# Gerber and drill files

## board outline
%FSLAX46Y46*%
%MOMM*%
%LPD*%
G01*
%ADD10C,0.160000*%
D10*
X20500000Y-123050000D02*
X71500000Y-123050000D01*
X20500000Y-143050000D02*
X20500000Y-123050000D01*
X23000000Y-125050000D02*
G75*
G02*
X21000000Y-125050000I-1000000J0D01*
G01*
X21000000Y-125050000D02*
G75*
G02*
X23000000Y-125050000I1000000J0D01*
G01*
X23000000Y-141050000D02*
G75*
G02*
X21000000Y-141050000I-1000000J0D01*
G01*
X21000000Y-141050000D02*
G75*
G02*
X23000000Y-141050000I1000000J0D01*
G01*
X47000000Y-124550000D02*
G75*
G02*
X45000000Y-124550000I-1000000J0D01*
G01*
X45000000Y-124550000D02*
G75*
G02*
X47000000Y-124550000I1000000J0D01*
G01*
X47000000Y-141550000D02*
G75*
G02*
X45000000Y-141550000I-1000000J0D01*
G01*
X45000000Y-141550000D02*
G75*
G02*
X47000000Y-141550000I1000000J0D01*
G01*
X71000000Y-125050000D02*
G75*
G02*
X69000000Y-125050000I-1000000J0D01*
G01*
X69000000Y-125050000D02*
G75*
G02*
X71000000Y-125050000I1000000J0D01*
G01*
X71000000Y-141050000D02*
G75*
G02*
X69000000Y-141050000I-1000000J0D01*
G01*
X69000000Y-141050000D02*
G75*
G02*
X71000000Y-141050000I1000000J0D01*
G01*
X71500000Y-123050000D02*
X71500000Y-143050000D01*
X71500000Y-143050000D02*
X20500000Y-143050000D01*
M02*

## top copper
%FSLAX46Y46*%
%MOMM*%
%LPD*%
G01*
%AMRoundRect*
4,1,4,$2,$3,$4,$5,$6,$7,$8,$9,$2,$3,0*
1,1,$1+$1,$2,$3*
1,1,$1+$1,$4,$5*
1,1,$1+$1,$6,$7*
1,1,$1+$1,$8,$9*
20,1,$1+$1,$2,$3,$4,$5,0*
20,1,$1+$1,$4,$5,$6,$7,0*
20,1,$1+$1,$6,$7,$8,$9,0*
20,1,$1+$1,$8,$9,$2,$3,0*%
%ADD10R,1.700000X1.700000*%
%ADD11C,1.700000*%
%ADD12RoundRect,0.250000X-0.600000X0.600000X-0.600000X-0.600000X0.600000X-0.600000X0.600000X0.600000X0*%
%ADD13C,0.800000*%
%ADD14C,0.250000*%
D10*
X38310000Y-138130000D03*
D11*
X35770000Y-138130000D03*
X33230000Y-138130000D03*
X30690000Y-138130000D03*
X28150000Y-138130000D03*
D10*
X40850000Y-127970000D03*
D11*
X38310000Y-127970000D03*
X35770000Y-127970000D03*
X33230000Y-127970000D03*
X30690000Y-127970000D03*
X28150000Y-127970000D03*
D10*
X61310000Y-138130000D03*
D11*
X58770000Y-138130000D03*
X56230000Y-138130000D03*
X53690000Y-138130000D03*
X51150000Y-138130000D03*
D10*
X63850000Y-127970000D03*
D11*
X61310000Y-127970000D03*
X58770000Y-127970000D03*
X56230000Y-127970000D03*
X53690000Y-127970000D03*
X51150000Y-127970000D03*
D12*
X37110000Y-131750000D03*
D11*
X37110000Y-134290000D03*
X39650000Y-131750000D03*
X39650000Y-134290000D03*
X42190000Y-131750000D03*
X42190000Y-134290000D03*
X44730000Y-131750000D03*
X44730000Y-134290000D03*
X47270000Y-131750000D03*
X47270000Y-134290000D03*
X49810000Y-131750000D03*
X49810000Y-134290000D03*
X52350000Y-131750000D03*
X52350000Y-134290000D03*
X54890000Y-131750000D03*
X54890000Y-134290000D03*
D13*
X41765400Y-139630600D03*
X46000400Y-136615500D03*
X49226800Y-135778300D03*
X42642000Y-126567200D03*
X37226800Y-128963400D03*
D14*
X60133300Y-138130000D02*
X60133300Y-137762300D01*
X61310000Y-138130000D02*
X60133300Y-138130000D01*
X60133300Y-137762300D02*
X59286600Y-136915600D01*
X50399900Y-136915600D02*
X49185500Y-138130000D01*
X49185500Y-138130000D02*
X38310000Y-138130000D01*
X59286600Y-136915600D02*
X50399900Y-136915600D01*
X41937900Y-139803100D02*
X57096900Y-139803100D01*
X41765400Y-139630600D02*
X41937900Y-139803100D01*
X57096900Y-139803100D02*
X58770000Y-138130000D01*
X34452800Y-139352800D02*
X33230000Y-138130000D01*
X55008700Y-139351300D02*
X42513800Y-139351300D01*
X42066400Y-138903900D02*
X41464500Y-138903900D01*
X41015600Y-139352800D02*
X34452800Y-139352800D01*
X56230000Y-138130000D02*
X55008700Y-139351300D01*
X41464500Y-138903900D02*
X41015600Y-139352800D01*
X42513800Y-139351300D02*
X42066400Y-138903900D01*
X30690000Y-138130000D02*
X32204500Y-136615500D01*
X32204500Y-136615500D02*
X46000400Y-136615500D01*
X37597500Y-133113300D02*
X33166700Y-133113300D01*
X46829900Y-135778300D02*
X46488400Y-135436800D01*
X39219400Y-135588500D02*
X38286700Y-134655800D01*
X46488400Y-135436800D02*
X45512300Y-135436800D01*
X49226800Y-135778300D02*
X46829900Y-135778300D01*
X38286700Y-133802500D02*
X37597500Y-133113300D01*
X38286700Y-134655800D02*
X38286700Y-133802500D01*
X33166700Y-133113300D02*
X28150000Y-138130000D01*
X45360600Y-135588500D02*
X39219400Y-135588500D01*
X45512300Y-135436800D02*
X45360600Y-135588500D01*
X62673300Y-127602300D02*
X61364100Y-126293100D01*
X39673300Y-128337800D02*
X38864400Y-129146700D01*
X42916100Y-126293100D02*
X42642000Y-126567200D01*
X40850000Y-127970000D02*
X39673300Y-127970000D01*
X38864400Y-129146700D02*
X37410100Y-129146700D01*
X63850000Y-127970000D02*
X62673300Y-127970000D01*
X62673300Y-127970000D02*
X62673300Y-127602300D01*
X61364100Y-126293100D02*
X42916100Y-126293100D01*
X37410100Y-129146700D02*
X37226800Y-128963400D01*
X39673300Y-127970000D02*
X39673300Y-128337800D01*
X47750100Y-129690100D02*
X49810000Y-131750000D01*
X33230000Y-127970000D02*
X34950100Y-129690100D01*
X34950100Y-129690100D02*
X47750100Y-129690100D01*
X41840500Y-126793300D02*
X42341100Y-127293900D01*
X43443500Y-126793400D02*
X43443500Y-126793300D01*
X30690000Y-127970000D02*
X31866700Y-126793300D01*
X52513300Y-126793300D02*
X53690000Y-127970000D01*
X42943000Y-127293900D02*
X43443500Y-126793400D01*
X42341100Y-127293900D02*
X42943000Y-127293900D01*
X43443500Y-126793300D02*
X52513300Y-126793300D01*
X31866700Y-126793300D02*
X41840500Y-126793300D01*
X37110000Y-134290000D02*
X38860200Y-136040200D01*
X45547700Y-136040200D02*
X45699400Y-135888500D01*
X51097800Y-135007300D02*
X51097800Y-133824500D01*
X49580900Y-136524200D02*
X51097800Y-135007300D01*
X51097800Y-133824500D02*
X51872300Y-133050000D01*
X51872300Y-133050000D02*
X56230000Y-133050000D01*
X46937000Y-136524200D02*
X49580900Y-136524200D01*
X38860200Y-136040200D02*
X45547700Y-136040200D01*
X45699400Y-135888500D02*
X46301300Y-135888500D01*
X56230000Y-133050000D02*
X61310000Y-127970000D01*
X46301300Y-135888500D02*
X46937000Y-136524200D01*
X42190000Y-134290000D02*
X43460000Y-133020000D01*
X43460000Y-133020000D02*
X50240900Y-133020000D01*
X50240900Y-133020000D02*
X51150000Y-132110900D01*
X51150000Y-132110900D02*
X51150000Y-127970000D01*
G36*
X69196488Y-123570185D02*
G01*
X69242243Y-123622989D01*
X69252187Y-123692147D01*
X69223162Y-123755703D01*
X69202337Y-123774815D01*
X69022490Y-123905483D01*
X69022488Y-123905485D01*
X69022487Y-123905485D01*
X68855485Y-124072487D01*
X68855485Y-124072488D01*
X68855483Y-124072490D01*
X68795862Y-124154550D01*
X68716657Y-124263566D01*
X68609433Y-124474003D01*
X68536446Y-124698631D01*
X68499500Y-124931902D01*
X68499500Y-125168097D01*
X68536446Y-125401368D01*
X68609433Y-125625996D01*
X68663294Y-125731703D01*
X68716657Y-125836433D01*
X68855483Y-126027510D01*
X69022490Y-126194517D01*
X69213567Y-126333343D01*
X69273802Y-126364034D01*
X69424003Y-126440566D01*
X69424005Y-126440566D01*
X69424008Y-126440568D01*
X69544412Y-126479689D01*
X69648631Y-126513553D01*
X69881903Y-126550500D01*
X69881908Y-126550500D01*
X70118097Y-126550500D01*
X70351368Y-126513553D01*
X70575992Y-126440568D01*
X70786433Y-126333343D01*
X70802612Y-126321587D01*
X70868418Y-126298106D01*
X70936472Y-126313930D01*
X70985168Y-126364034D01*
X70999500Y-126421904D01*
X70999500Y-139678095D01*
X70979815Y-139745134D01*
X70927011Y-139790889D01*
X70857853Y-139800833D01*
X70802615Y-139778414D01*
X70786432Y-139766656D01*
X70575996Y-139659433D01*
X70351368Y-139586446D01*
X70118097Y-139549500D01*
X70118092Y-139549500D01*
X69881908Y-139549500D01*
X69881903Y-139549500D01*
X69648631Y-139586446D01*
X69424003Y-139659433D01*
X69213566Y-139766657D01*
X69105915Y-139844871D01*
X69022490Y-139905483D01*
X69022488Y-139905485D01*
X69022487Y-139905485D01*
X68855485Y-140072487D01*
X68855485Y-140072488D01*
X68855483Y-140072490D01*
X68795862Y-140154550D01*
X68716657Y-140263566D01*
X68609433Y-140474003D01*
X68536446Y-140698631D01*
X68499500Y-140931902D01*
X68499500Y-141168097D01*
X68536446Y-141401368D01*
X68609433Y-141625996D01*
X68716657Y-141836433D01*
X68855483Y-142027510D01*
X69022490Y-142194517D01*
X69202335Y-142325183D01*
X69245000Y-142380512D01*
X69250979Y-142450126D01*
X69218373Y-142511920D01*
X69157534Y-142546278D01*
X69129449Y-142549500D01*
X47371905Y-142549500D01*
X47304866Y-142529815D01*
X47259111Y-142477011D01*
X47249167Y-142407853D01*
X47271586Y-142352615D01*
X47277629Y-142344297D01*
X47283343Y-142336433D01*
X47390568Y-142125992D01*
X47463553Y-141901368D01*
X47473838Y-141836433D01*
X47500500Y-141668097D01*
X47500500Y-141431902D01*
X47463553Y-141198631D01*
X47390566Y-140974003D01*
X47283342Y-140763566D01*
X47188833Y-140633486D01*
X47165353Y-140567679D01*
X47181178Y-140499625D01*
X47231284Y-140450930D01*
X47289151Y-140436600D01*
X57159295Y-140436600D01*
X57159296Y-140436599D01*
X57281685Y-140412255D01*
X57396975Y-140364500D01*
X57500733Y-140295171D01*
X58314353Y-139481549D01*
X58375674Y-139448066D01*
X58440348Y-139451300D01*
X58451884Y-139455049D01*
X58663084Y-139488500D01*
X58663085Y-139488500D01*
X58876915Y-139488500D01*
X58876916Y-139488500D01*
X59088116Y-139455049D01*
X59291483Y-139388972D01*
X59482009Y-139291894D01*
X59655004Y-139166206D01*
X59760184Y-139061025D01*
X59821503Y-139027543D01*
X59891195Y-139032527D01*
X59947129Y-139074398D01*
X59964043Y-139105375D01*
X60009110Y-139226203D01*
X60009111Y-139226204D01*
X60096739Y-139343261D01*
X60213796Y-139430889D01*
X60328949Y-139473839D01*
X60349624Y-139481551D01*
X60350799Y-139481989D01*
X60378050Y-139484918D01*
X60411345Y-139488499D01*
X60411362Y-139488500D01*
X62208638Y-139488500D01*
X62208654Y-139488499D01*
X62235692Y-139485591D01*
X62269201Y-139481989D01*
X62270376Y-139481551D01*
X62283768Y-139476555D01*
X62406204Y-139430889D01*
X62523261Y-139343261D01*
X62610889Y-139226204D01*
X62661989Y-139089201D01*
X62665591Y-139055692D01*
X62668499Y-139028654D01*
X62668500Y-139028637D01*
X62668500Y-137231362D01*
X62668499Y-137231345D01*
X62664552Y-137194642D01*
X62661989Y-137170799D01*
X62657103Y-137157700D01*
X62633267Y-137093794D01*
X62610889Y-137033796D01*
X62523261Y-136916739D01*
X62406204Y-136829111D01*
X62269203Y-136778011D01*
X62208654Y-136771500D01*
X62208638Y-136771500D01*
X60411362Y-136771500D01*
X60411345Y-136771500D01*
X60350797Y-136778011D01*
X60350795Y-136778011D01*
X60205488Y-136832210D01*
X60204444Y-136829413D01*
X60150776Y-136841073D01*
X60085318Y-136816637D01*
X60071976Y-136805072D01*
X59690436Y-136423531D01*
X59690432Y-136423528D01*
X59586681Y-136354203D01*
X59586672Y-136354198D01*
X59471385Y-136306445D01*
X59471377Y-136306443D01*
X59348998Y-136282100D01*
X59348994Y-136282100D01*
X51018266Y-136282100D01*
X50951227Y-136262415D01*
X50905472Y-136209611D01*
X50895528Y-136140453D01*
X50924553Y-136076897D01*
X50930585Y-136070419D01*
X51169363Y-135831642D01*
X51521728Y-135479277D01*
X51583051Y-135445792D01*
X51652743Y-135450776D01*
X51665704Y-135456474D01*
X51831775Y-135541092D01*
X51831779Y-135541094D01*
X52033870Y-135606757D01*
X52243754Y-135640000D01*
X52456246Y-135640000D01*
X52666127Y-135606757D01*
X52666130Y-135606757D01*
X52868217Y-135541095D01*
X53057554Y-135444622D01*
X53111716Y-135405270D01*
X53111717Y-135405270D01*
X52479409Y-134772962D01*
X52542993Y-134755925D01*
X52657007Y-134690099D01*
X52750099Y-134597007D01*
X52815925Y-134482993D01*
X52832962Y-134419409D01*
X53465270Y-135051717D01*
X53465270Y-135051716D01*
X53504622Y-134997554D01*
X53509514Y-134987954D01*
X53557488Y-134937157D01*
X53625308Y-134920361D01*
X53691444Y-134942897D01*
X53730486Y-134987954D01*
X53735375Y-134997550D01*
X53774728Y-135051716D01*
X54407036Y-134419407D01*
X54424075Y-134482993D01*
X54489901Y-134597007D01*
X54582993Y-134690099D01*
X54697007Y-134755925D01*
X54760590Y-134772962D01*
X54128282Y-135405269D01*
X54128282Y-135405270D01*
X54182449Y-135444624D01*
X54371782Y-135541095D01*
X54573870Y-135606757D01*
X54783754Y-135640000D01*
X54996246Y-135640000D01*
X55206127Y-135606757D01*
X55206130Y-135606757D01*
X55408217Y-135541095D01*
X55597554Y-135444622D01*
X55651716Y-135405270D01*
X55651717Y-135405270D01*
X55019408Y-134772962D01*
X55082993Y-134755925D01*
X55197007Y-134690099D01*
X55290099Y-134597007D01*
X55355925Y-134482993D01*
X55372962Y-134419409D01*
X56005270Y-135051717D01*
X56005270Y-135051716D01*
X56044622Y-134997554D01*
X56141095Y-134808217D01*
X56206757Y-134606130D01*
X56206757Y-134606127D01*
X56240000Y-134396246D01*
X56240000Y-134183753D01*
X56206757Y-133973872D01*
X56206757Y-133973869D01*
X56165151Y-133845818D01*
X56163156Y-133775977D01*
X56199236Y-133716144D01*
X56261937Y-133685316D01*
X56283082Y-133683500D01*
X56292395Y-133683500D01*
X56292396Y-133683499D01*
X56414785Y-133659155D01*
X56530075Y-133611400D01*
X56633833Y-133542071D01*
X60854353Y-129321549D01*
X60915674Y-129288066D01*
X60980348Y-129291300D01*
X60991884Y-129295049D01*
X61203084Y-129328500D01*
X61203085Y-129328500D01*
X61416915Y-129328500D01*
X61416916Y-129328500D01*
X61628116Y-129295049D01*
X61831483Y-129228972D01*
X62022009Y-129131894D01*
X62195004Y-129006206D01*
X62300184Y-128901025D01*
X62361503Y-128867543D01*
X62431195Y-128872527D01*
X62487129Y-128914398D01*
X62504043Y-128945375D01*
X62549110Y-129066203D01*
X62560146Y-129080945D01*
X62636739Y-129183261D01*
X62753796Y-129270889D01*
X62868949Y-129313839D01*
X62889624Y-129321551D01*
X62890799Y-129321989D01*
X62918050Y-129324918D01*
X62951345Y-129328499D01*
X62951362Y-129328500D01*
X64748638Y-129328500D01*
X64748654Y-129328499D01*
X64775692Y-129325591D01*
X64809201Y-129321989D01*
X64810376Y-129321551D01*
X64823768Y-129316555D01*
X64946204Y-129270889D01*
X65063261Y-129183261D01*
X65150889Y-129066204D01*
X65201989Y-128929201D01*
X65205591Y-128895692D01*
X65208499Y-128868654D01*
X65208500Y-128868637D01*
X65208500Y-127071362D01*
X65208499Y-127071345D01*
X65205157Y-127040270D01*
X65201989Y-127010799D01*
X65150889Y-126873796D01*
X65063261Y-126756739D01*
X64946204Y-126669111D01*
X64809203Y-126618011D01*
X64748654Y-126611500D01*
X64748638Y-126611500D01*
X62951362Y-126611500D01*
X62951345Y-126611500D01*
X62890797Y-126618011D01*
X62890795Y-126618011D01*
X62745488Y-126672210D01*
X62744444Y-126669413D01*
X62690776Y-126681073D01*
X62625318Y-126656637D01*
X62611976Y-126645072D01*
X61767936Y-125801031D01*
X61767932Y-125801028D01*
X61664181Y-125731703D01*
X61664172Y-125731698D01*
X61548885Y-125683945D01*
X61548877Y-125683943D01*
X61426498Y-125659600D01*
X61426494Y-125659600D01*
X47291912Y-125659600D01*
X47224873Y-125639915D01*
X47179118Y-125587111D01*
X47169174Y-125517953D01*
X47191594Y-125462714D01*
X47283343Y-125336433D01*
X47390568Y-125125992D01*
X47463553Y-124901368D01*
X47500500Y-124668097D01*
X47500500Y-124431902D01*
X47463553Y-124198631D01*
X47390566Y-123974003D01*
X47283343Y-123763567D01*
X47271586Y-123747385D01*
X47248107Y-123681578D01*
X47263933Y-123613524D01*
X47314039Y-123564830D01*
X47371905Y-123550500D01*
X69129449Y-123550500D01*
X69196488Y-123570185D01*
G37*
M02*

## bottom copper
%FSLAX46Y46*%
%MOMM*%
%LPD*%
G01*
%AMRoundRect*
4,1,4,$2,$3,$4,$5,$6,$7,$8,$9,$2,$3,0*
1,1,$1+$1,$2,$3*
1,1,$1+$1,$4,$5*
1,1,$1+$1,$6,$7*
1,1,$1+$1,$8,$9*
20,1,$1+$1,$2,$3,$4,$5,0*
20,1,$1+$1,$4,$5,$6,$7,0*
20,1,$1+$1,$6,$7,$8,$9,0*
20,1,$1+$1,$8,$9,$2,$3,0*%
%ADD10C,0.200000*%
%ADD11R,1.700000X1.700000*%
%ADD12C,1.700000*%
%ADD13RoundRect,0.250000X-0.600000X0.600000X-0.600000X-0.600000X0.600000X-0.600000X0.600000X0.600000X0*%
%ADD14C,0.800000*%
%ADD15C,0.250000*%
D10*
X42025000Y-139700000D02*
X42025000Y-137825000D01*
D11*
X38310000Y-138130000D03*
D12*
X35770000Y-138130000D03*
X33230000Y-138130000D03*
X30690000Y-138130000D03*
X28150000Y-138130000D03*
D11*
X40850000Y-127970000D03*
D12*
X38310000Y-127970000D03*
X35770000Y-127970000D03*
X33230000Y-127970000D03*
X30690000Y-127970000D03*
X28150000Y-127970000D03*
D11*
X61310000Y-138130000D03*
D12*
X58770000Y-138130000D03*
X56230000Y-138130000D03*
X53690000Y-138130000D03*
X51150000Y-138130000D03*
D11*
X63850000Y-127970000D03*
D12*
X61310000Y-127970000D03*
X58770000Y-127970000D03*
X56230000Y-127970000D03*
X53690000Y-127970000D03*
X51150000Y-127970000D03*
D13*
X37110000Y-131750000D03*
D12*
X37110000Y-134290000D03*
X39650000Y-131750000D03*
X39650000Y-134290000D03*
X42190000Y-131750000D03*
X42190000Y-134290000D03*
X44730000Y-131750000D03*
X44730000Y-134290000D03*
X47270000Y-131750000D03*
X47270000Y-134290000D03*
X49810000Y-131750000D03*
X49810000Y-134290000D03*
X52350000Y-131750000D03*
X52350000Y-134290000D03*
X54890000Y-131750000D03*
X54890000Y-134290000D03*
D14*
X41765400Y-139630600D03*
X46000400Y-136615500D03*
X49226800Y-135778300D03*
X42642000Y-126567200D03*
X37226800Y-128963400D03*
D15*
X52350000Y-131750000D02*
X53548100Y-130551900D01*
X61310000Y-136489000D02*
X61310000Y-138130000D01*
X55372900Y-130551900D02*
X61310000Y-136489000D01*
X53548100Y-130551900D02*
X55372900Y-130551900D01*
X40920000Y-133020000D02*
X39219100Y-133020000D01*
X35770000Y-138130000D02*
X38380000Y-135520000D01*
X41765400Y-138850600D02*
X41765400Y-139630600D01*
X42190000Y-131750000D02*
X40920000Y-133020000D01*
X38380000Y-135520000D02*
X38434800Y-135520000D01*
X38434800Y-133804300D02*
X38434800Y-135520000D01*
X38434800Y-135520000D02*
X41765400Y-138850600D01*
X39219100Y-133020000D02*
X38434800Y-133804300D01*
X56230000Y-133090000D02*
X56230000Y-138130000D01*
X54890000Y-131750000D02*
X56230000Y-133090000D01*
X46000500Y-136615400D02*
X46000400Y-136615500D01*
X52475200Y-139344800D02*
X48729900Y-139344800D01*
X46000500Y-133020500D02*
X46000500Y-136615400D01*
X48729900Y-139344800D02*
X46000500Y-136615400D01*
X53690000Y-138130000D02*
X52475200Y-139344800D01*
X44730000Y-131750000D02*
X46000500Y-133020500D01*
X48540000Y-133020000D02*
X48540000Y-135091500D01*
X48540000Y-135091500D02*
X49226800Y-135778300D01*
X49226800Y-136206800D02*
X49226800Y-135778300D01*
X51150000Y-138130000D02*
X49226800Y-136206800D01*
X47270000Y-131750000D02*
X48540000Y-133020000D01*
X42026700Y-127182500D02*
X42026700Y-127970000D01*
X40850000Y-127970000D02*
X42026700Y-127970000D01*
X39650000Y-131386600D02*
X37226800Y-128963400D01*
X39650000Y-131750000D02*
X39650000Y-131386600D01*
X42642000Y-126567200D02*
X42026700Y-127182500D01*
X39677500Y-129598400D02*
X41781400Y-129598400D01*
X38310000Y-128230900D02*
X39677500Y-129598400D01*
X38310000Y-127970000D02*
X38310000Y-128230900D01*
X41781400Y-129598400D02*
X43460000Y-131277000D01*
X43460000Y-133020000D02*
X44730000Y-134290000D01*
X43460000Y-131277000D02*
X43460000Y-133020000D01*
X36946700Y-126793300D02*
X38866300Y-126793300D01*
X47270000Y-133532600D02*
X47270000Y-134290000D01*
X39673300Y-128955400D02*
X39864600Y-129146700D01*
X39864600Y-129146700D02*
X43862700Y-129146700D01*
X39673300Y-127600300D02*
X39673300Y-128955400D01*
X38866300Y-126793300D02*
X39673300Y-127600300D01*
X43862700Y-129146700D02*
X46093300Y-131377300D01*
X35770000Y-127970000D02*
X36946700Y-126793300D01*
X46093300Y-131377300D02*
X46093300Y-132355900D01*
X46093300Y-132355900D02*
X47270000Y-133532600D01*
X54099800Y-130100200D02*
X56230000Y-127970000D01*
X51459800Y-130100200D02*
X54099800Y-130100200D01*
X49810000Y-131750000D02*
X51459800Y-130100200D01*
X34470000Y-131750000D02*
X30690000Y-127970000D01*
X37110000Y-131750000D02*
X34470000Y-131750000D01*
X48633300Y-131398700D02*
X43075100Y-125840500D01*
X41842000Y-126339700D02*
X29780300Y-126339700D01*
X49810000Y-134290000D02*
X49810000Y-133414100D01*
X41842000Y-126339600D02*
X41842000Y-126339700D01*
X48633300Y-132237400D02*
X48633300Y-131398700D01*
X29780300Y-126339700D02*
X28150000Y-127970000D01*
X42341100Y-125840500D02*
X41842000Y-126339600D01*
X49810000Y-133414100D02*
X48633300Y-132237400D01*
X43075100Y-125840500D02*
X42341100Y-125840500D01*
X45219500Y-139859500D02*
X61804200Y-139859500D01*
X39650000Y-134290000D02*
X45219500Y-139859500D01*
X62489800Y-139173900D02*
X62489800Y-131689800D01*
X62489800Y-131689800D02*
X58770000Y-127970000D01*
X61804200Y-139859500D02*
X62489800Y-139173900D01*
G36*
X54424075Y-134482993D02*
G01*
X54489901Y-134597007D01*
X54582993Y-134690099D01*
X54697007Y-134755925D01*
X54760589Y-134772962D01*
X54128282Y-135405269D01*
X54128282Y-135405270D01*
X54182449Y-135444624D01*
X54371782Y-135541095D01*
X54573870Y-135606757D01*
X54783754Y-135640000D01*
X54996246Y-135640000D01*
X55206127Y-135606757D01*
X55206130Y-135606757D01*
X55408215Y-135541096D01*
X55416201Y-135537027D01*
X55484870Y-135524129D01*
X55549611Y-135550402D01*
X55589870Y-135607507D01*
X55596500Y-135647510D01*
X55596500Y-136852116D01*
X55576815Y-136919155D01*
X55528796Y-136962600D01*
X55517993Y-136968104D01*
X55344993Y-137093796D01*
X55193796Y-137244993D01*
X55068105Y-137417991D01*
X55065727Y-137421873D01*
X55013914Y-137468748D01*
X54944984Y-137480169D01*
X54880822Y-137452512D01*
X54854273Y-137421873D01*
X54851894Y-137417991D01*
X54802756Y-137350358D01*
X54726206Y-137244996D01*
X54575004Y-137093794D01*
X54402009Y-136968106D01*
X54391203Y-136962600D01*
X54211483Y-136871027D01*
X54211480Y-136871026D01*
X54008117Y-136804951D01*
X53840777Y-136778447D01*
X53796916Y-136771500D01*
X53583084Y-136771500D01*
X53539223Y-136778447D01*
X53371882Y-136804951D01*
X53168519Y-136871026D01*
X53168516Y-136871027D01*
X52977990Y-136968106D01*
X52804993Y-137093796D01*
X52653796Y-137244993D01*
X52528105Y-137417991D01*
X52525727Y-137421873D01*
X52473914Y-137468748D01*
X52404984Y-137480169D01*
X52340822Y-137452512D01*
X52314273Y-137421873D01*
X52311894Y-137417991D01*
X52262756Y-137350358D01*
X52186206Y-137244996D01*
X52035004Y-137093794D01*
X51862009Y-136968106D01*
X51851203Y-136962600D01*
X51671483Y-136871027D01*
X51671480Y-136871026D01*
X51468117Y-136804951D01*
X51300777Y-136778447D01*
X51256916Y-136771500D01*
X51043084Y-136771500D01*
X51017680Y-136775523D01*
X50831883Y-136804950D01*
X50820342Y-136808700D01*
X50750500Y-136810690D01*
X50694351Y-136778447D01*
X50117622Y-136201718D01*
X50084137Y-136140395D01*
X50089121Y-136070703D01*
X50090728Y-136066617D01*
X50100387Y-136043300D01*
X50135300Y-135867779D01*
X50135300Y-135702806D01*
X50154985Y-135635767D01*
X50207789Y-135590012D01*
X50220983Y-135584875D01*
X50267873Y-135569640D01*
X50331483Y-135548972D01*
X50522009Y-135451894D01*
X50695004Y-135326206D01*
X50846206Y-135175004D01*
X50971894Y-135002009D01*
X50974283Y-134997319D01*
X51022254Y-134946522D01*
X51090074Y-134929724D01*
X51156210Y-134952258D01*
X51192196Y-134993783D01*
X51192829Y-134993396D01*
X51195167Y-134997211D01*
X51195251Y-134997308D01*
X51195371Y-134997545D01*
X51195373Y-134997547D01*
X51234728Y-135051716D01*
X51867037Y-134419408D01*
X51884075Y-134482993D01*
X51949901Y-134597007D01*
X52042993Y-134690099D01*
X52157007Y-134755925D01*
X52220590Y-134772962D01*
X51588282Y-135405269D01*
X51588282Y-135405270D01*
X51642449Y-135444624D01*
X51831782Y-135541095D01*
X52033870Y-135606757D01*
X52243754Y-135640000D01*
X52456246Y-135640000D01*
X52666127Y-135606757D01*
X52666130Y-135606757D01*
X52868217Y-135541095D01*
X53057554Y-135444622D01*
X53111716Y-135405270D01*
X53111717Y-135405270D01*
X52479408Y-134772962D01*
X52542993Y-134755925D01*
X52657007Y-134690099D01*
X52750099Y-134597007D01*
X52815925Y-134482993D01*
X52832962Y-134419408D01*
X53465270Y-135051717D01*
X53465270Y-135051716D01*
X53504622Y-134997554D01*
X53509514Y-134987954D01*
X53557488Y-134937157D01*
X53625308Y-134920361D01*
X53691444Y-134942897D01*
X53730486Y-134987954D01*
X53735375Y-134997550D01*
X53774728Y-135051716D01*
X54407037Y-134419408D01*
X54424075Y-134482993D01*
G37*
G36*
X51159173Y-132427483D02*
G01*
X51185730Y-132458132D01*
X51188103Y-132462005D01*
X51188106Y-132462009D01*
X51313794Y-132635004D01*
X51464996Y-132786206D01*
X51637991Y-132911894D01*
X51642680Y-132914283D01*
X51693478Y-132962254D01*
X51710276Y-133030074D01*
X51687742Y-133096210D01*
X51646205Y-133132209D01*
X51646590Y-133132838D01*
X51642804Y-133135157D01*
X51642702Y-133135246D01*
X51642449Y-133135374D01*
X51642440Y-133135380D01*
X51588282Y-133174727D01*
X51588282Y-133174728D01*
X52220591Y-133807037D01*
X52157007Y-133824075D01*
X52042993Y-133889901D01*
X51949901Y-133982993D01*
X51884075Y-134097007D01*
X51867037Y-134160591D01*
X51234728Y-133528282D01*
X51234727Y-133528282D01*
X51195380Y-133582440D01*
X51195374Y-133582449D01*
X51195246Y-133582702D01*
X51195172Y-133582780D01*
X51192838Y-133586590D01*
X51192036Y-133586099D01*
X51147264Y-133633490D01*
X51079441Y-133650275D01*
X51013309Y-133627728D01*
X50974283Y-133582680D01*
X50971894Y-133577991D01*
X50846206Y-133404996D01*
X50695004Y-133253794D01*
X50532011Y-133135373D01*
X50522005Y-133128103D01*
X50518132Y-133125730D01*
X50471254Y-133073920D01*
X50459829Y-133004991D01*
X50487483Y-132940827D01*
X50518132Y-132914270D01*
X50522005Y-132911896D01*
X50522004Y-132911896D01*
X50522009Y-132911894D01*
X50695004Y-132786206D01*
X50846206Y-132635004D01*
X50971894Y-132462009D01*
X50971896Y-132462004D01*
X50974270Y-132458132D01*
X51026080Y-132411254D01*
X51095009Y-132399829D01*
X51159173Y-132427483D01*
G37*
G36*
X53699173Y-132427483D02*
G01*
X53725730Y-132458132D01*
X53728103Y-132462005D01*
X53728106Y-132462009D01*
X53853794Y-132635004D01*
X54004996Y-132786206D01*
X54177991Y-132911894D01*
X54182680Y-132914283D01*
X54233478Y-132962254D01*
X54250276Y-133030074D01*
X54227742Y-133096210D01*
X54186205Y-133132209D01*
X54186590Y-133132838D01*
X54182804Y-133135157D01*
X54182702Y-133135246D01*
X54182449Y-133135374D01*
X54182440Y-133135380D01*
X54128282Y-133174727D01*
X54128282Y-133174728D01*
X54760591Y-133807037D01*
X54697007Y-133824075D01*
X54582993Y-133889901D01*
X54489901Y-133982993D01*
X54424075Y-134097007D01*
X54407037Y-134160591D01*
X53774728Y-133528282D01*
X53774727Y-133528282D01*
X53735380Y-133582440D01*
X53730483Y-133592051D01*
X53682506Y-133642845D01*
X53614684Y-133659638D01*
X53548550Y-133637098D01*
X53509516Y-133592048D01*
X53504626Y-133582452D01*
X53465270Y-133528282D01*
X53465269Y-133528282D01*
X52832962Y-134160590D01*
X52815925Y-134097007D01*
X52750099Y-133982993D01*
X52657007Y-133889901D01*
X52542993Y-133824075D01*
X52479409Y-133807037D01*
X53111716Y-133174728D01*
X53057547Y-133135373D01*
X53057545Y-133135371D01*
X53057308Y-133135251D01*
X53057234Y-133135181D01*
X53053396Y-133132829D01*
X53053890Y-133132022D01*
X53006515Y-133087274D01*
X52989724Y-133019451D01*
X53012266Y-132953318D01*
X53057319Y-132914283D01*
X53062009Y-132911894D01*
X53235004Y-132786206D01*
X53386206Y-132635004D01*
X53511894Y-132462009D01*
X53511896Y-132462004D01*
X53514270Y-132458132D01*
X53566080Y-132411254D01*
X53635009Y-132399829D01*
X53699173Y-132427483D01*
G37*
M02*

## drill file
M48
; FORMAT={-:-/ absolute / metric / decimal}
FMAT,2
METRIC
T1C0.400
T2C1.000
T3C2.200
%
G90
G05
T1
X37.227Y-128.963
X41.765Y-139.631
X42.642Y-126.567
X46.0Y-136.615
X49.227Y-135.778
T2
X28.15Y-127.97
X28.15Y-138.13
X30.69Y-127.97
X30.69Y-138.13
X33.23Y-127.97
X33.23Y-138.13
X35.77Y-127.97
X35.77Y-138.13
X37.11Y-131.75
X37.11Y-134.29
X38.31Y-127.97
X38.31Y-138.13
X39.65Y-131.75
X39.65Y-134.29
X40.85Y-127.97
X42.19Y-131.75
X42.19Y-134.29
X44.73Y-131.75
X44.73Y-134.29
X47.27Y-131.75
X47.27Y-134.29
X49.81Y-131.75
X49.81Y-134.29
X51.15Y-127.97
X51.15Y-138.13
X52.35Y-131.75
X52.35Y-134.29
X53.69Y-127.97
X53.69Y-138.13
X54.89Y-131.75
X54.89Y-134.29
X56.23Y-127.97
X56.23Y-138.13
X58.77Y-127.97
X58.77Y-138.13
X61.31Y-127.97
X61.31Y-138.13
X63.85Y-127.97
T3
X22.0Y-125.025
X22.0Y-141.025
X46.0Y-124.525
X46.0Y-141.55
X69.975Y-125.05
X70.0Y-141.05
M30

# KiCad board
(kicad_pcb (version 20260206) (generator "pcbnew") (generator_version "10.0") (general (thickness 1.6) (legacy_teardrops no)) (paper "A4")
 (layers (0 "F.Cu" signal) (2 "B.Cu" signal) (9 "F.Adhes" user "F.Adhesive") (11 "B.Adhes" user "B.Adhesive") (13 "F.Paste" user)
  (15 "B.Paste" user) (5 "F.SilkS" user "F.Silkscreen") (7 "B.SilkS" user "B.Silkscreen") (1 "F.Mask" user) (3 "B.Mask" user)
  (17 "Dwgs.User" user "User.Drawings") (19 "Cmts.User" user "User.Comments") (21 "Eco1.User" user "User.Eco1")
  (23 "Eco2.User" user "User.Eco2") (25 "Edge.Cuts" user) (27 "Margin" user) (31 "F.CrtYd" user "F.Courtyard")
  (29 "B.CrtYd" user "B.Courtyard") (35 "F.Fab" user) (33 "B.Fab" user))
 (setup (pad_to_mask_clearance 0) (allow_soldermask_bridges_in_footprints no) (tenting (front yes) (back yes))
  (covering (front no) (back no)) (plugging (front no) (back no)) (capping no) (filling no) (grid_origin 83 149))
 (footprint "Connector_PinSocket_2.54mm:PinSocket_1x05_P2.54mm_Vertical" (layer "F.Cu") (at 38.31 138.13 -90)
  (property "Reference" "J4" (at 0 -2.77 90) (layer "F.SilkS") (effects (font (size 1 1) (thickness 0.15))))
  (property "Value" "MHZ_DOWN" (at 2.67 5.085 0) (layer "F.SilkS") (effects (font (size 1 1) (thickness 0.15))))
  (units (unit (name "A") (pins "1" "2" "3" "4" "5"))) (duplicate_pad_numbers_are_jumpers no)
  (pad "1" thru_hole rect (at 0 0 270) (size 1.7 1.7) (drill 1) (layers "*.Cu" "*.Mask") (remove_unused_layers no) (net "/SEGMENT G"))
  (pad "2" thru_hole circle (at 0 2.54 270) (size 1.7 1.7) (drill 1) (layers "*.Cu" "*.Mask") (remove_unused_layers no) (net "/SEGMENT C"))
  (pad "3" thru_hole circle (at 0 5.08 270) (size 1.7 1.7) (drill 1) (layers "*.Cu" "*.Mask") (remove_unused_layers no) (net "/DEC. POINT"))
  (pad "4" thru_hole circle (at 0 7.62 270) (size 1.7 1.7) (drill 1) (layers "*.Cu" "*.Mask") (remove_unused_layers no) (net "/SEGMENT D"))
  (pad "5" thru_hole circle (at 0 10.16 270) (size 1.7 1.7) (drill 1) (layers "*.Cu" "*.Mask") (remove_unused_layers no) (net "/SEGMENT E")))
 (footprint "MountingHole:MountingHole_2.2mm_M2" (layer "F.Cu") (at 69.975 125.05)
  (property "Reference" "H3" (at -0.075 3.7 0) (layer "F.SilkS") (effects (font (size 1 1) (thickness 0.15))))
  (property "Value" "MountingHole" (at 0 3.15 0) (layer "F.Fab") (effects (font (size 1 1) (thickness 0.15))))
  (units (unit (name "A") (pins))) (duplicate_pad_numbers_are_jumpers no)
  (pad "" np_thru_hole circle (at 0 0) (size 2.2 2.2) (drill 2.2) (layers "*.Cu" "*.Mask")))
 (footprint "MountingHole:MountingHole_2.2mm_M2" (layer "F.Cu") (at 70 141.05)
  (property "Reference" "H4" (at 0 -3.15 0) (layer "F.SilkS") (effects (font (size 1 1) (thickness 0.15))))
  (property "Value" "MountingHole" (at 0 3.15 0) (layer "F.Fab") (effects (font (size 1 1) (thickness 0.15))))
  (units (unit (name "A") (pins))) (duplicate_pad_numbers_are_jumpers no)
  (pad "" np_thru_hole circle (at 0 0) (size 2.2 2.2) (drill 2.2) (layers "*.Cu" "*.Mask")))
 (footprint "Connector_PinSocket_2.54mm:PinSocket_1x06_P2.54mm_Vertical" (layer "F.Cu") (at 40.85 127.97 -90)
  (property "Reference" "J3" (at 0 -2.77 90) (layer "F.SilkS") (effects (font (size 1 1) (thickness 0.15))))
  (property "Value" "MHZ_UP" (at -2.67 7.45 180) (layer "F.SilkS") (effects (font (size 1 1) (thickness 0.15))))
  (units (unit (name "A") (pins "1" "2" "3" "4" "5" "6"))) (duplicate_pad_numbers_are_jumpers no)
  (pad "1" thru_hole rect (at 0 0 270) (size 1.7 1.7) (drill 1) (layers "*.Cu" "*.Mask") (remove_unused_layers no) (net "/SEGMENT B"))
  (pad "2" thru_hole circle (at 0 2.54 270) (size 1.7 1.7) (drill 1) (layers "*.Cu" "*.Mask") (remove_unused_layers no) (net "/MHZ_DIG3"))
  (pad "3" thru_hole circle (at 0 5.08 270) (size 1.7 1.7) (drill 1) (layers "*.Cu" "*.Mask") (remove_unused_layers no) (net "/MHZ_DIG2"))
  (pad "4" thru_hole circle (at 0 7.62 270) (size 1.7 1.7) (drill 1) (layers "*.Cu" "*.Mask") (remove_unused_layers no) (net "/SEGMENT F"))
  (pad "5" thru_hole circle (at 0 10.16 270) (size 1.7 1.7) (drill 1) (layers "*.Cu" "*.Mask") (remove_unused_layers no) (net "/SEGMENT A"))
  (pad "6" thru_hole circle (at 0 12.7 270) (size 1.7 1.7) (drill 1) (layers "*.Cu" "*.Mask") (remove_unused_layers no) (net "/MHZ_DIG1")))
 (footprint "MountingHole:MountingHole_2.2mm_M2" (layer "F.Cu") (at 46 141.55 180)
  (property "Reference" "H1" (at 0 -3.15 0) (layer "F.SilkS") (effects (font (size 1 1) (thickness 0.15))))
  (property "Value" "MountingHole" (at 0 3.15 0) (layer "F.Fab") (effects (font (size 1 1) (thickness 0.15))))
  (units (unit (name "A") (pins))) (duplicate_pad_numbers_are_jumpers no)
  (pad "" np_thru_hole circle (at 0 0 180) (size 2.2 2.2) (drill 2.2) (layers "*.Cu" "*.Mask")))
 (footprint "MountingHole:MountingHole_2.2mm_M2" (layer "F.Cu") (at 22 125.025)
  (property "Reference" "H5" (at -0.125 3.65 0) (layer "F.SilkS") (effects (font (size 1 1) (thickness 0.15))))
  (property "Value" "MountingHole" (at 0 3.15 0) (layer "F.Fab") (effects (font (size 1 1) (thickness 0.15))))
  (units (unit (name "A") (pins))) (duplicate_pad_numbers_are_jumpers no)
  (pad "" np_thru_hole circle (at 0 0) (size 2.2 2.2) (drill 2.2) (layers "*.Cu" "*.Mask")))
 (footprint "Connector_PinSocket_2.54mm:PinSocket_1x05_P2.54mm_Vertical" (layer "F.Cu") (at 61.31 138.13 -90)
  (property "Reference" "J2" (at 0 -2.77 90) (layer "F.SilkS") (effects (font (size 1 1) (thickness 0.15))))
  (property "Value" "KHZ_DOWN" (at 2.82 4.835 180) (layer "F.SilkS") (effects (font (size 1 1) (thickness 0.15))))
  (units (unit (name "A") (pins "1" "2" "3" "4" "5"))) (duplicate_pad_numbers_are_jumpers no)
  (pad "1" thru_hole rect (at 0 0 270) (size 1.7 1.7) (drill 1) (layers "*.Cu" "*.Mask") (remove_unused_layers no) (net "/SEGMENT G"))
  (pad "2" thru_hole circle (at 0 2.54 270) (size 1.7 1.7) (drill 1) (layers "*.Cu" "*.Mask") (remove_unused_layers no) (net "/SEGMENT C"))
  (pad "3" thru_hole circle (at 0 5.08 270) (size 1.7 1.7) (drill 1) (layers "*.Cu" "*.Mask") (remove_unused_layers no) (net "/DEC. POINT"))
  (pad "4" thru_hole circle (at 0 7.62 270) (size 1.7 1.7) (drill 1) (layers "*.Cu" "*.Mask") (remove_unused_layers no) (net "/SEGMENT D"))
  (pad "5" thru_hole circle (at 0 10.16 270) (size 1.7 1.7) (drill 1) (layers "*.Cu" "*.Mask") (remove_unused_layers no) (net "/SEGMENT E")))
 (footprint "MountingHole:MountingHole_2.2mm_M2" (layer "F.Cu") (at 46 124.525 180)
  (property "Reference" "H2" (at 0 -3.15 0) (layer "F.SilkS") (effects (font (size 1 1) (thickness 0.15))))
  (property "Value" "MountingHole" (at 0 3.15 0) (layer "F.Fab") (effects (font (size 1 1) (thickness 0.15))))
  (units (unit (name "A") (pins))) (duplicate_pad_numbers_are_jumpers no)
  (pad "" np_thru_hole circle (at 0 0 180) (size 2.2 2.2) (drill 2.2) (layers "*.Cu" "*.Mask")))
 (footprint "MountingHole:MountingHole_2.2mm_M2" (layer "F.Cu") (at 22 141.025)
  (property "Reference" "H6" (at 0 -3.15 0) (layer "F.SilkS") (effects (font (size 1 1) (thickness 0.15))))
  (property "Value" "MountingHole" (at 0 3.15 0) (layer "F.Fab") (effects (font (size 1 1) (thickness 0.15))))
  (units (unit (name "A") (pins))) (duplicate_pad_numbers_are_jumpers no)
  (pad "" np_thru_hole circle (at 0 0) (size 2.2 2.2) (drill 2.2) (layers "*.Cu" "*.Mask")))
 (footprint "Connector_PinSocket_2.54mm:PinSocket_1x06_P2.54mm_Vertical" (layer "F.Cu") (at 63.85 127.97 -90)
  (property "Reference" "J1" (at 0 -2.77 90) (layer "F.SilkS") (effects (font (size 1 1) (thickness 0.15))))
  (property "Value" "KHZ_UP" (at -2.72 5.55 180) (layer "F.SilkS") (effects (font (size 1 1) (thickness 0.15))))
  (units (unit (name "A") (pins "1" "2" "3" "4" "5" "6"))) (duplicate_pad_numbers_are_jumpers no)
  (pad "1" thru_hole rect (at 0 0 270) (size 1.7 1.7) (drill 1) (layers "*.Cu" "*.Mask") (remove_unused_layers no) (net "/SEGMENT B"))
  (pad "2" thru_hole circle (at 0 2.54 270) (size 1.7 1.7) (drill 1) (layers "*.Cu" "*.Mask") (remove_unused_layers no) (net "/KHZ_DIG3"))
  (pad "3" thru_hole circle (at 0 5.08 270) (size 1.7 1.7) (drill 1) (layers "*.Cu" "*.Mask") (remove_unused_layers no) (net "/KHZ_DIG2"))
  (pad "4" thru_hole circle (at 0 7.62 270) (size 1.7 1.7) (drill 1) (layers "*.Cu" "*.Mask") (remove_unused_layers no) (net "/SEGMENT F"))
  (pad "5" thru_hole circle (at 0 10.16 270) (size 1.7 1.7) (drill 1) (layers "*.Cu" "*.Mask") (remove_unused_layers no) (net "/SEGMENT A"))
  (pad "6" thru_hole circle (at 0 12.7 270) (size 1.7 1.7) (drill 1) (layers "*.Cu" "*.Mask") (remove_unused_layers no) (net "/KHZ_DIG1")))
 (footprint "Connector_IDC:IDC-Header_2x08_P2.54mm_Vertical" (layer "B.Cu") (at 37.11 131.75 -90)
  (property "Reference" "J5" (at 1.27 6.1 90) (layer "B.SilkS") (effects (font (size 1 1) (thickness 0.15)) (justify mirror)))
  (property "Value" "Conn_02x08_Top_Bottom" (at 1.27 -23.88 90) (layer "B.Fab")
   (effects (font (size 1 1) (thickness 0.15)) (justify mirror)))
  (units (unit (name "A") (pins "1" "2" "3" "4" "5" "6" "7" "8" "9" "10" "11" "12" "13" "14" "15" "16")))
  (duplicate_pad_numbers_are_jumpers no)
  (pad "1" thru_hole roundrect (at 0 0 270) (size 1.7 1.7) (drill 1) (layers "*.Cu" "*.Mask") (remove_unused_layers no)
   (roundrect_rratio 0.147059) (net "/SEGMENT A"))
  (pad "2" thru_hole circle (at 2.54 0 270) (size 1.7 1.7) (drill 1) (layers "*.Cu" "*.Mask") (remove_unused_layers no) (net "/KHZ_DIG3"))
  (pad "3" thru_hole circle (at 0 -2.54 270) (size 1.7 1.7) (drill 1) (layers "*.Cu" "*.Mask") (remove_unused_layers no) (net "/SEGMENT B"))
  (pad "4" thru_hole circle (at 2.54 -2.54 270) (size 1.7 1.7) (drill 1) (layers "*.Cu" "*.Mask") (remove_unused_layers no)
   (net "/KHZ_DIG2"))
  (pad "5" thru_hole circle (at 0 -5.08 270) (size 1.7 1.7) (drill 1) (layers "*.Cu" "*.Mask") (remove_unused_layers no) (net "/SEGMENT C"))
  (pad "6" thru_hole circle (at 2.54 -5.08 270) (size 1.7 1.7) (drill 1) (layers "*.Cu" "*.Mask") (remove_unused_layers no)
   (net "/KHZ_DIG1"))
  (pad "7" thru_hole circle (at 0 -7.62 270) (size 1.7 1.7) (drill 1) (layers "*.Cu" "*.Mask") (remove_unused_layers no) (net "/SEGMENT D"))
  (pad "8" thru_hole circle (at 2.54 -7.62 270) (size 1.7 1.7) (drill 1) (layers "*.Cu" "*.Mask") (remove_unused_layers no)
   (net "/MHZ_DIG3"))
  (pad "9" thru_hole circle (at 0 -10.16 270) (size 1.7 1.7) (drill 1) (layers "*.Cu" "*.Mask") (remove_unused_layers no) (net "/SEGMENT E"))
  (pad "10" thru_hole circle (at 2.54 -10.16 270) (size 1.7 1.7) (drill 1) (layers "*.Cu" "*.Mask") (remove_unused_layers no)
   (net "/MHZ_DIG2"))
  (pad "11" thru_hole circle (at 0 -12.7 270) (size 1.7 1.7) (drill 1) (layers "*.Cu" "*.Mask") (remove_unused_layers no) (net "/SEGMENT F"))
  (pad "12" thru_hole circle (at 2.54 -12.7 270) (size 1.7 1.7) (drill 1) (layers "*.Cu" "*.Mask") (remove_unused_layers no)
   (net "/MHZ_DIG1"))
  (pad "13" thru_hole circle (at 0 -15.24 270) (size 1.7 1.7) (drill 1) (layers "*.Cu" "*.Mask") (remove_unused_layers no)
   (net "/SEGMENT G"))
  (pad "14" thru_hole circle (at 2.54 -15.24 270) (size 1.7 1.7) (drill 1) (layers "*.Cu" "*.Mask") (remove_unused_layers no) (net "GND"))
  (pad "15" thru_hole circle (at 0 -17.78 270) (size 1.7 1.7) (drill 1) (layers "*.Cu" "*.Mask") (remove_unused_layers no)
   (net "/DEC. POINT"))
  (pad "16" thru_hole circle (at 2.54 -17.78 270) (size 1.7 1.7) (drill 1) (layers "*.Cu" "*.Mask") (remove_unused_layers no) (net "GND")))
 (gr_line (start 42.025 139.7) (end 42.025 137.825) (stroke (width 0.2) (type default)) (layer "B.Cu") (net "/SEGMENT C"))
 (gr_line (start 20.5 123.05) (end 71.5 123.05) (stroke (width 0.16) (type solid)) (layer "Edge.Cuts"))
 (gr_line (start 20.5 143.05) (end 20.5 123.05) (stroke (width 0.16) (type solid)) (layer "Edge.Cuts"))
 (gr_circle (center 22 125.05) (end 23 125.05) (stroke (width 0.16) (type solid)) (fill no) (layer "Edge.Cuts"))
 (gr_circle (center 22 141.05) (end 23 141.05) (stroke (width 0.16) (type solid)) (fill no) (layer "Edge.Cuts"))
 (gr_circle (center 46 124.55) (end 47 124.55) (stroke (width 0.16) (type solid)) (fill no) (layer "Edge.Cuts"))
 (gr_circle (center 46 141.55) (end 47 141.55) (stroke (width 0.16) (type solid)) (fill no) (layer "Edge.Cuts"))
 (gr_circle (center 70 125.05) (end 71 125.05) (stroke (width 0.16) (type solid)) (fill no) (layer "Edge.Cuts"))
 (gr_circle (center 70 141.05) (end 71 141.05) (stroke (width 0.16) (type solid)) (fill no) (layer "Edge.Cuts"))
 (gr_line (start 71.5 123.05) (end 71.5 143.05) (stroke (width 0.16) (type solid)) (layer "Edge.Cuts"))
 (gr_line (start 71.5 143.05) (end 20.5 143.05) (stroke (width 0.16) (type solid)) (layer "Edge.Cuts"))
 (segment (start 60.1333 138.13) (end 60.1333 137.7623) (width 0.25) (layer "F.Cu") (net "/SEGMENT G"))
 (segment (start 61.31 138.13) (end 60.1333 138.13) (width 0.25) (layer "F.Cu") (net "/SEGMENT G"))
 (segment (start 60.1333 137.7623) (end 59.2866 136.9156) (width 0.25) (layer "F.Cu") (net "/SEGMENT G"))
 (segment (start 50.3999 136.9156) (end 49.1855 138.13) (width 0.25) (layer "F.Cu") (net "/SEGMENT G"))
 (segment (start 49.1855 138.13) (end 38.31 138.13) (width 0.25) (layer "F.Cu") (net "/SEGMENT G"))
 (segment (start 59.2866 136.9156) (end 50.3999 136.9156) (width 0.25) (layer "F.Cu") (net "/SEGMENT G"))
 (segment (start 52.35 131.75) (end 53.5481 130.5519) (width 0.25) (layer "B.Cu") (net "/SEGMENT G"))
 (segment (start 61.31 136.489) (end 61.31 138.13) (width 0.25) (layer "B.Cu") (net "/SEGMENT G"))
 (segment (start 55.3729 130.5519) (end 61.31 136.489) (width 0.25) (layer "B.Cu") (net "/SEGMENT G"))
 (segment (start 53.5481 130.5519) (end 55.3729 130.5519) (width 0.25) (layer "B.Cu") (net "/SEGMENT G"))
 (segment (start 41.9379 139.8031) (end 57.0969 139.8031) (width 0.25) (layer "F.Cu") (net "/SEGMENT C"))
 (segment (start 41.7654 139.6306) (end 41.9379 139.8031) (width 0.25) (layer "F.Cu") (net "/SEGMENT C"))
 (segment (start 57.0969 139.8031) (end 58.77 138.13) (width 0.25) (layer "F.Cu") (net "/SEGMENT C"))
 (via (at 41.7654 139.6306) (size 0.8) (drill 0.4) (layers "F.Cu" "B.Cu") (capping no) (covering (front no) (back no))
  (plugging (front no) (back no)) (filling no) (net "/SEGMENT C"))
 (segment (start 40.92 133.02) (end 39.2191 133.02) (width 0.25) (layer "B.Cu") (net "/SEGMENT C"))
 (segment (start 35.77 138.13) (end 38.38 135.52) (width 0.25) (layer "B.Cu") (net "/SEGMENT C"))
 (segment (start 41.7654 138.8506) (end 41.7654 139.6306) (width 0.25) (layer "B.Cu") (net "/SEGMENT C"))
 (segment (start 42.19 131.75) (end 40.92 133.02) (width 0.25) (layer "B.Cu") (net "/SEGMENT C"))
 (segment (start 38.38 135.52) (end 38.4348 135.52) (width 0.25) (layer "B.Cu") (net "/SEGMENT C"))
 (segment (start 38.4348 133.8043) (end 38.4348 135.52) (width 0.25) (layer "B.Cu") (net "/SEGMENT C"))
 (segment (start 38.4348 135.52) (end 41.7654 138.8506) (width 0.25) (layer "B.Cu") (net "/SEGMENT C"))
 (segment (start 39.2191 133.02) (end 38.4348 133.8043) (width 0.25) (layer "B.Cu") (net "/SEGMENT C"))
 (segment (start 34.4528 139.3528) (end 33.23 138.13) (width 0.25) (layer "F.Cu") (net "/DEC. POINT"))
 (segment (start 55.0087 139.3513) (end 42.5138 139.3513) (width 0.25) (layer "F.Cu") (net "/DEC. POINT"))
 (segment (start 42.0664 138.9039) (end 41.4645 138.9039) (width 0.25) (layer "F.Cu") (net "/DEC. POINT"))
 (segment (start 41.0156 139.3528) (end 34.4528 139.3528) (width 0.25) (layer "F.Cu") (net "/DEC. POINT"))
 (segment (start 56.23 138.13) (end 55.0087 139.3513) (width 0.25) (layer "F.Cu") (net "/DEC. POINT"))
 (segment (start 41.4645 138.9039) (end 41.0156 139.3528) (width 0.25) (layer "F.Cu") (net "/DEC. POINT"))
 (segment (start 42.5138 139.3513) (end 42.0664 138.9039) (width 0.25) (layer "F.Cu") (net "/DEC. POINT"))
 (segment (start 56.23 133.09) (end 56.23 138.13) (width 0.25) (layer "B.Cu") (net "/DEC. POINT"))
 (segment (start 54.89 131.75) (end 56.23 133.09) (width 0.25) (layer "B.Cu") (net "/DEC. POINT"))
 (segment (start 30.69 138.13) (end 32.2045 136.6155) (width 0.25) (layer "F.Cu") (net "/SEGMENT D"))
 (segment (start 32.2045 136.6155) (end 46.0004 136.6155) (width 0.25) (layer "F.Cu") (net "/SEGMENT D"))
 (via (at 46.0004 136.6155) (size 0.8) (drill 0.4) (layers "F.Cu" "B.Cu") (capping no) (covering (front no) (back no))
  (plugging (front no) (back no)) (filling no) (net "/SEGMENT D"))
 (segment (start 46.0005 136.6154) (end 46.0004 136.6155) (width 0.25) (layer "B.Cu") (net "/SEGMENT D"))
 (segment (start 52.4752 139.3448) (end 48.7299 139.3448) (width 0.25) (layer "B.Cu") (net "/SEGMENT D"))
 (segment (start 46.0005 133.0205) (end 46.0005 136.6154) (width 0.25) (layer "B.Cu") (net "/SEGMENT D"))
 (segment (start 48.7299 139.3448) (end 46.0005 136.6154) (width 0.25) (layer "B.Cu") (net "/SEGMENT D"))
 (segment (start 53.69 138.13) (end 52.4752 139.3448) (width 0.25) (layer "B.Cu") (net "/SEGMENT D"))
 (segment (start 44.73 131.75) (end 46.0005 133.0205) (width 0.25) (layer "B.Cu") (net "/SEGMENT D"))
 (segment (start 37.5975 133.1133) (end 33.1667 133.1133) (width 0.25) (layer "F.Cu") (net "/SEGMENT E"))
 (segment (start 46.8299 135.7783) (end 46.4884 135.4368) (width 0.25) (layer "F.Cu") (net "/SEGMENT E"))
 (segment (start 39.2194 135.5885) (end 38.2867 134.6558) (width 0.25) (layer "F.Cu") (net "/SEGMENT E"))
 (segment (start 46.4884 135.4368) (end 45.5123 135.4368) (width 0.25) (layer "F.Cu") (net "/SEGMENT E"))
 (segment (start 49.2268 135.7783) (end 46.8299 135.7783) (width 0.25) (layer "F.Cu") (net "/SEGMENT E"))
 (segment (start 38.2867 133.8025) (end 37.5975 133.1133) (width 0.25) (layer "F.Cu") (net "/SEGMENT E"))
 (segment (start 38.2867 134.6558) (end 38.2867 133.8025) (width 0.25) (layer "F.Cu") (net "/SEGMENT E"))
 (segment (start 33.1667 133.1133) (end 28.15 138.13) (width 0.25) (layer "F.Cu") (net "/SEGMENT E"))
 (segment (start 45.3606 135.5885) (end 39.2194 135.5885) (width 0.25) (layer "F.Cu") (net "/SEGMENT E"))
 (segment (start 45.5123 135.4368) (end 45.3606 135.5885) (width 0.25) (layer "F.Cu") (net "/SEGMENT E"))
 (via (at 49.2268 135.7783) (size 0.8) (drill 0.4) (layers "F.Cu" "B.Cu") (capping no) (covering (front no) (back no))
  (plugging (front no) (back no)) (filling no) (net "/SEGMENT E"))
 (segment (start 48.54 133.02) (end 48.54 135.0915) (width 0.25) (layer "B.Cu") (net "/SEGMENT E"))
 (segment (start 48.54 135.0915) (end 49.2268 135.7783) (width 0.25) (layer "B.Cu") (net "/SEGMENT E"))
 (segment (start 49.2268 136.2068) (end 49.2268 135.7783) (width 0.25) (layer "B.Cu") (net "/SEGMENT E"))
 (segment (start 51.15 138.13) (end 49.2268 136.2068) (width 0.25) (layer "B.Cu") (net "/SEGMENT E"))
 (segment (start 47.27 131.75) (end 48.54 133.02) (width 0.25) (layer "B.Cu") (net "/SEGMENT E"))
 (segment (start 62.6733 127.6023) (end 61.3641 126.2931) (width 0.25) (layer "F.Cu") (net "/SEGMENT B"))
 (segment (start 39.6733 128.3378) (end 38.8644 129.1467) (width 0.25) (layer "F.Cu") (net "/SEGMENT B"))
 (segment (start 42.9161 126.2931) (end 42.642 126.5672) (width 0.25) (layer "F.Cu") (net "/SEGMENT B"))
 (segment (start 40.85 127.97) (end 39.6733 127.97) (width 0.25) (layer "F.Cu") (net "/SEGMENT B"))
 (segment (start 38.8644 129.1467) (end 37.4101 129.1467) (width 0.25) (layer "F.Cu") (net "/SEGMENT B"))
 (segment (start 63.85 127.97) (end 62.6733 127.97) (width 0.25) (layer "F.Cu") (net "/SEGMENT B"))
 (segment (start 62.6733 127.97) (end 62.6733 127.6023) (width 0.25) (layer "F.Cu") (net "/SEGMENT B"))
 (segment (start 61.3641 126.2931) (end 42.9161 126.2931) (width 0.25) (layer "F.Cu") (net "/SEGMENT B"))
 (segment (start 37.4101 129.1467) (end 37.2268 128.9634) (width 0.25) (layer "F.Cu") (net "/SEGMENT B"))
 (segment (start 39.6733 127.97) (end 39.6733 128.3378) (width 0.25) (layer "F.Cu") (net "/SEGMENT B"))
 (via (at 42.642 126.5672) (size 0.8) (drill 0.4) (layers "F.Cu" "B.Cu") (capping no) (covering (front no) (back no))
  (plugging (front no) (back no)) (filling no) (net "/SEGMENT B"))
 (via (at 37.2268 128.9634) (size 0.8) (drill 0.4) (layers "F.Cu" "B.Cu") (capping no) (covering (front no) (back no))
  (plugging (front no) (back no)) (filling no) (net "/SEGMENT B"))
 (segment (start 42.0267 127.1825) (end 42.0267 127.97) (width 0.25) (layer "B.Cu") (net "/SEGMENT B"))
 (segment (start 40.85 127.97) (end 42.0267 127.97) (width 0.25) (layer "B.Cu") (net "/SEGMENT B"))
 (segment (start 39.65 131.3866) (end 37.2268 128.9634) (width 0.25) (layer "B.Cu") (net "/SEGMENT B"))
 (segment (start 39.65 131.75) (end 39.65 131.3866) (width 0.25) (layer "B.Cu") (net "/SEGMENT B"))
 (segment (start 42.642 126.5672) (end 42.0267 127.1825) (width 0.25) (layer "B.Cu") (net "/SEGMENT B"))
 (segment (start 39.6775 129.5984) (end 41.7814 129.5984) (width 0.25) (layer "B.Cu") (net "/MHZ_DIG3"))
 (segment (start 38.31 128.2309) (end 39.6775 129.5984) (width 0.25) (layer "B.Cu") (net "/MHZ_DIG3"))
 (segment (start 38.31 127.97) (end 38.31 128.2309) (width 0.25) (layer "B.Cu") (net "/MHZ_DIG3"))
 (segment (start 41.7814 129.5984) (end 43.46 131.277) (width 0.25) (layer "B.Cu") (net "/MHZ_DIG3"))
 (segment (start 43.46 133.02) (end 44.73 134.29) (width 0.25) (layer "B.Cu") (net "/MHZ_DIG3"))
 (segment (start 43.46 131.277) (end 43.46 133.02) (width 0.25) (layer "B.Cu") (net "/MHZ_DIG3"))
 (segment (start 36.9467 126.7933) (end 38.8663 126.7933) (width 0.25) (layer "B.Cu") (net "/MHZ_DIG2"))
 (segment (start 47.27 133.5326) (end 47.27 134.29) (width 0.25) (layer "B.Cu") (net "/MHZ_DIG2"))
 (segment (start 39.6733 128.9554) (end 39.8646 129.1467) (width 0.25) (layer "B.Cu") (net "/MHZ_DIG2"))
 (segment (start 39.8646 129.1467) (end 43.8627 129.1467) (width 0.25) (layer "B.Cu") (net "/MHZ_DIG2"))
 (segment (start 39.6733 127.6003) (end 39.6733 128.9554) (width 0.25) (layer "B.Cu") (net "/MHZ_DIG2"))
 (segment (start 38.8663 126.7933) (end 39.6733 127.6003) (width 0.25) (layer "B.Cu") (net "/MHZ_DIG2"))
 (segment (start 43.8627 129.1467) (end 46.0933 131.3773) (width 0.25) (layer "B.Cu") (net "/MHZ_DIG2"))
 (segment (start 35.77 127.97) (end 36.9467 126.7933) (width 0.25) (layer "B.Cu") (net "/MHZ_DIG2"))
 (segment (start 46.0933 131.3773) (end 46.0933 132.3559) (width 0.25) (layer "B.Cu") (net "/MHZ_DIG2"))
 (segment (start 46.0933 132.3559) (end 47.27 133.5326) (width 0.25) (layer "B.Cu") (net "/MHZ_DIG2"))
 (segment (start 47.7501 129.6901) (end 49.81 131.75) (width 0.25) (layer "F.Cu") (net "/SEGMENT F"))
 (segment (start 33.23 127.97) (end 34.9501 129.6901) (width 0.25) (layer "F.Cu") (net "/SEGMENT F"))
 (segment (start 34.9501 129.6901) (end 47.7501 129.6901) (width 0.25) (layer "F.Cu") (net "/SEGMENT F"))
 (segment (start 54.0998 130.1002) (end 56.23 127.97) (width 0.25) (layer "B.Cu") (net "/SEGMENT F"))
 (segment (start 51.4598 130.1002) (end 54.0998 130.1002) (width 0.25) (layer "B.Cu") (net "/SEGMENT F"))
 (segment (start 49.81 131.75) (end 51.4598 130.1002) (width 0.25) (layer "B.Cu") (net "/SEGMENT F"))
 (segment (start 41.8405 126.7933) (end 42.3411 127.2939) (width 0.25) (layer "F.Cu") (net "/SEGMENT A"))
 (segment (start 43.4435 126.7934) (end 43.4435 126.7933) (width 0.25) (layer "F.Cu") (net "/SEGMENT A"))
 (segment (start 30.69 127.97) (end 31.8667 126.7933) (width 0.25) (layer "F.Cu") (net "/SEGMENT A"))
 (segment (start 52.5133 126.7933) (end 53.69 127.97) (width 0.25) (layer "F.Cu") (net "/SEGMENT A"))
 (segment (start 42.943 127.2939) (end 43.4435 126.7934) (width 0.25) (layer "F.Cu") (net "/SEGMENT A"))
 (segment (start 42.3411 127.2939) (end 42.943 127.2939) (width 0.25) (layer "F.Cu") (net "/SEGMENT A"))
 (segment (start 43.4435 126.7933) (end 52.5133 126.7933) (width 0.25) (layer "F.Cu") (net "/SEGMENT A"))
 (segment (start 31.8667 126.7933) (end 41.8405 126.7933) (width 0.25) (layer "F.Cu") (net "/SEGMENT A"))
 (segment (start 34.47 131.75) (end 30.69 127.97) (width 0.25) (layer "B.Cu") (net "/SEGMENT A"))
 (segment (start 37.11 131.75) (end 34.47 131.75) (width 0.25) (layer "B.Cu") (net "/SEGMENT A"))
 (segment (start 48.6333 131.3987) (end 43.0751 125.8405) (width 0.25) (layer "B.Cu") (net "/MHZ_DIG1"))
 (segment (start 41.842 126.3397) (end 29.7803 126.3397) (width 0.25) (layer "B.Cu") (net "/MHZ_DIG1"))
 (segment (start 49.81 134.29) (end 49.81 133.4141) (width 0.25) (layer "B.Cu") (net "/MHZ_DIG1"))
 (segment (start 41.842 126.3396) (end 41.842 126.3397) (width 0.25) (layer "B.Cu") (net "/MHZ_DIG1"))
 (segment (start 48.6333 132.2374) (end 48.6333 131.3987) (width 0.25) (layer "B.Cu") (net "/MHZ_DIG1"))
 (segment (start 29.7803 126.3397) (end 28.15 127.97) (width 0.25) (layer "B.Cu") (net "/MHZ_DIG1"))
 (segment (start 42.3411 125.8405) (end 41.842 126.3396) (width 0.25) (layer "B.Cu") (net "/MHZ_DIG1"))
 (segment (start 49.81 133.4141) (end 48.6333 132.2374) (width 0.25) (layer "B.Cu") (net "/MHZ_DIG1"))
 (segment (start 43.0751 125.8405) (end 42.3411 125.8405) (width 0.25) (layer "B.Cu") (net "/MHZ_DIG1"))
 (segment (start 37.11 134.29) (end 38.8602 136.0402) (width 0.25) (layer "F.Cu") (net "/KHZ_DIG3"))
 (segment (start 45.5477 136.0402) (end 45.6994 135.8885) (width 0.25) (layer "F.Cu") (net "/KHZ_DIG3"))
 (segment (start 51.0978 135.0073) (end 51.0978 133.8245) (width 0.25) (layer "F.Cu") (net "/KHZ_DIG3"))
 (segment (start 49.5809 136.5242) (end 51.0978 135.0073) (width 0.25) (layer "F.Cu") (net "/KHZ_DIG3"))
 (segment (start 51.0978 133.8245) (end 51.8723 133.05) (width 0.25) (layer "F.Cu") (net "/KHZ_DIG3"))
 (segment (start 51.8723 133.05) (end 56.23 133.05) (width 0.25) (layer "F.Cu") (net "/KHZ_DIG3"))
 (segment (start 46.937 136.5242) (end 49.5809 136.5242) (width 0.25) (layer "F.Cu") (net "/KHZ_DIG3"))
 (segment (start 38.8602 136.0402) (end 45.5477 136.0402) (width 0.25) (layer "F.Cu") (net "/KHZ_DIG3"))
 (segment (start 45.6994 135.8885) (end 46.3013 135.8885) (width 0.25) (layer "F.Cu") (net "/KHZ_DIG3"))
 (segment (start 56.23 133.05) (end 61.31 127.97) (width 0.25) (layer "F.Cu") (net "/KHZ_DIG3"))
 (segment (start 46.3013 135.8885) (end 46.937 136.5242) (width 0.25) (layer "F.Cu") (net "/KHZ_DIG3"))
 (segment (start 45.2195 139.8595) (end 61.8042 139.8595) (width 0.25) (layer "B.Cu") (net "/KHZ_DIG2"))
 (segment (start 39.65 134.29) (end 45.2195 139.8595) (width 0.25) (layer "B.Cu") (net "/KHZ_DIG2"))
 (segment (start 62.4898 139.1739) (end 62.4898 131.6898) (width 0.25) (layer "B.Cu") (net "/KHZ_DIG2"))
 (segment (start 62.4898 131.6898) (end 58.77 127.97) (width 0.25) (layer "B.Cu") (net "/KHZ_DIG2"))
 (segment (start 61.8042 139.8595) (end 62.4898 139.1739) (width 0.25) (layer "B.Cu") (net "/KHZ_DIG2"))
 (segment (start 42.19 134.29) (end 43.46 133.02) (width 0.25) (layer "F.Cu") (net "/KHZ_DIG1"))
 (segment (start 43.46 133.02) (end 50.2409 133.02) (width 0.25) (layer "F.Cu") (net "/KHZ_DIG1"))
 (segment (start 50.2409 133.02) (end 51.15 132.1109) (width 0.25) (layer "F.Cu") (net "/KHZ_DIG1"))
 (segment (start 51.15 132.1109) (end 51.15 127.97) (width 0.25) (layer "F.Cu") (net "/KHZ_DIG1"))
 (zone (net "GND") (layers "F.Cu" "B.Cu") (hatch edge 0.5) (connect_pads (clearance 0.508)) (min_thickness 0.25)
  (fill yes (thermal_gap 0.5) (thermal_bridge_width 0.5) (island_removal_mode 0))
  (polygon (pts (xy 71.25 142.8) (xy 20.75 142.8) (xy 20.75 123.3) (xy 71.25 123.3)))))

